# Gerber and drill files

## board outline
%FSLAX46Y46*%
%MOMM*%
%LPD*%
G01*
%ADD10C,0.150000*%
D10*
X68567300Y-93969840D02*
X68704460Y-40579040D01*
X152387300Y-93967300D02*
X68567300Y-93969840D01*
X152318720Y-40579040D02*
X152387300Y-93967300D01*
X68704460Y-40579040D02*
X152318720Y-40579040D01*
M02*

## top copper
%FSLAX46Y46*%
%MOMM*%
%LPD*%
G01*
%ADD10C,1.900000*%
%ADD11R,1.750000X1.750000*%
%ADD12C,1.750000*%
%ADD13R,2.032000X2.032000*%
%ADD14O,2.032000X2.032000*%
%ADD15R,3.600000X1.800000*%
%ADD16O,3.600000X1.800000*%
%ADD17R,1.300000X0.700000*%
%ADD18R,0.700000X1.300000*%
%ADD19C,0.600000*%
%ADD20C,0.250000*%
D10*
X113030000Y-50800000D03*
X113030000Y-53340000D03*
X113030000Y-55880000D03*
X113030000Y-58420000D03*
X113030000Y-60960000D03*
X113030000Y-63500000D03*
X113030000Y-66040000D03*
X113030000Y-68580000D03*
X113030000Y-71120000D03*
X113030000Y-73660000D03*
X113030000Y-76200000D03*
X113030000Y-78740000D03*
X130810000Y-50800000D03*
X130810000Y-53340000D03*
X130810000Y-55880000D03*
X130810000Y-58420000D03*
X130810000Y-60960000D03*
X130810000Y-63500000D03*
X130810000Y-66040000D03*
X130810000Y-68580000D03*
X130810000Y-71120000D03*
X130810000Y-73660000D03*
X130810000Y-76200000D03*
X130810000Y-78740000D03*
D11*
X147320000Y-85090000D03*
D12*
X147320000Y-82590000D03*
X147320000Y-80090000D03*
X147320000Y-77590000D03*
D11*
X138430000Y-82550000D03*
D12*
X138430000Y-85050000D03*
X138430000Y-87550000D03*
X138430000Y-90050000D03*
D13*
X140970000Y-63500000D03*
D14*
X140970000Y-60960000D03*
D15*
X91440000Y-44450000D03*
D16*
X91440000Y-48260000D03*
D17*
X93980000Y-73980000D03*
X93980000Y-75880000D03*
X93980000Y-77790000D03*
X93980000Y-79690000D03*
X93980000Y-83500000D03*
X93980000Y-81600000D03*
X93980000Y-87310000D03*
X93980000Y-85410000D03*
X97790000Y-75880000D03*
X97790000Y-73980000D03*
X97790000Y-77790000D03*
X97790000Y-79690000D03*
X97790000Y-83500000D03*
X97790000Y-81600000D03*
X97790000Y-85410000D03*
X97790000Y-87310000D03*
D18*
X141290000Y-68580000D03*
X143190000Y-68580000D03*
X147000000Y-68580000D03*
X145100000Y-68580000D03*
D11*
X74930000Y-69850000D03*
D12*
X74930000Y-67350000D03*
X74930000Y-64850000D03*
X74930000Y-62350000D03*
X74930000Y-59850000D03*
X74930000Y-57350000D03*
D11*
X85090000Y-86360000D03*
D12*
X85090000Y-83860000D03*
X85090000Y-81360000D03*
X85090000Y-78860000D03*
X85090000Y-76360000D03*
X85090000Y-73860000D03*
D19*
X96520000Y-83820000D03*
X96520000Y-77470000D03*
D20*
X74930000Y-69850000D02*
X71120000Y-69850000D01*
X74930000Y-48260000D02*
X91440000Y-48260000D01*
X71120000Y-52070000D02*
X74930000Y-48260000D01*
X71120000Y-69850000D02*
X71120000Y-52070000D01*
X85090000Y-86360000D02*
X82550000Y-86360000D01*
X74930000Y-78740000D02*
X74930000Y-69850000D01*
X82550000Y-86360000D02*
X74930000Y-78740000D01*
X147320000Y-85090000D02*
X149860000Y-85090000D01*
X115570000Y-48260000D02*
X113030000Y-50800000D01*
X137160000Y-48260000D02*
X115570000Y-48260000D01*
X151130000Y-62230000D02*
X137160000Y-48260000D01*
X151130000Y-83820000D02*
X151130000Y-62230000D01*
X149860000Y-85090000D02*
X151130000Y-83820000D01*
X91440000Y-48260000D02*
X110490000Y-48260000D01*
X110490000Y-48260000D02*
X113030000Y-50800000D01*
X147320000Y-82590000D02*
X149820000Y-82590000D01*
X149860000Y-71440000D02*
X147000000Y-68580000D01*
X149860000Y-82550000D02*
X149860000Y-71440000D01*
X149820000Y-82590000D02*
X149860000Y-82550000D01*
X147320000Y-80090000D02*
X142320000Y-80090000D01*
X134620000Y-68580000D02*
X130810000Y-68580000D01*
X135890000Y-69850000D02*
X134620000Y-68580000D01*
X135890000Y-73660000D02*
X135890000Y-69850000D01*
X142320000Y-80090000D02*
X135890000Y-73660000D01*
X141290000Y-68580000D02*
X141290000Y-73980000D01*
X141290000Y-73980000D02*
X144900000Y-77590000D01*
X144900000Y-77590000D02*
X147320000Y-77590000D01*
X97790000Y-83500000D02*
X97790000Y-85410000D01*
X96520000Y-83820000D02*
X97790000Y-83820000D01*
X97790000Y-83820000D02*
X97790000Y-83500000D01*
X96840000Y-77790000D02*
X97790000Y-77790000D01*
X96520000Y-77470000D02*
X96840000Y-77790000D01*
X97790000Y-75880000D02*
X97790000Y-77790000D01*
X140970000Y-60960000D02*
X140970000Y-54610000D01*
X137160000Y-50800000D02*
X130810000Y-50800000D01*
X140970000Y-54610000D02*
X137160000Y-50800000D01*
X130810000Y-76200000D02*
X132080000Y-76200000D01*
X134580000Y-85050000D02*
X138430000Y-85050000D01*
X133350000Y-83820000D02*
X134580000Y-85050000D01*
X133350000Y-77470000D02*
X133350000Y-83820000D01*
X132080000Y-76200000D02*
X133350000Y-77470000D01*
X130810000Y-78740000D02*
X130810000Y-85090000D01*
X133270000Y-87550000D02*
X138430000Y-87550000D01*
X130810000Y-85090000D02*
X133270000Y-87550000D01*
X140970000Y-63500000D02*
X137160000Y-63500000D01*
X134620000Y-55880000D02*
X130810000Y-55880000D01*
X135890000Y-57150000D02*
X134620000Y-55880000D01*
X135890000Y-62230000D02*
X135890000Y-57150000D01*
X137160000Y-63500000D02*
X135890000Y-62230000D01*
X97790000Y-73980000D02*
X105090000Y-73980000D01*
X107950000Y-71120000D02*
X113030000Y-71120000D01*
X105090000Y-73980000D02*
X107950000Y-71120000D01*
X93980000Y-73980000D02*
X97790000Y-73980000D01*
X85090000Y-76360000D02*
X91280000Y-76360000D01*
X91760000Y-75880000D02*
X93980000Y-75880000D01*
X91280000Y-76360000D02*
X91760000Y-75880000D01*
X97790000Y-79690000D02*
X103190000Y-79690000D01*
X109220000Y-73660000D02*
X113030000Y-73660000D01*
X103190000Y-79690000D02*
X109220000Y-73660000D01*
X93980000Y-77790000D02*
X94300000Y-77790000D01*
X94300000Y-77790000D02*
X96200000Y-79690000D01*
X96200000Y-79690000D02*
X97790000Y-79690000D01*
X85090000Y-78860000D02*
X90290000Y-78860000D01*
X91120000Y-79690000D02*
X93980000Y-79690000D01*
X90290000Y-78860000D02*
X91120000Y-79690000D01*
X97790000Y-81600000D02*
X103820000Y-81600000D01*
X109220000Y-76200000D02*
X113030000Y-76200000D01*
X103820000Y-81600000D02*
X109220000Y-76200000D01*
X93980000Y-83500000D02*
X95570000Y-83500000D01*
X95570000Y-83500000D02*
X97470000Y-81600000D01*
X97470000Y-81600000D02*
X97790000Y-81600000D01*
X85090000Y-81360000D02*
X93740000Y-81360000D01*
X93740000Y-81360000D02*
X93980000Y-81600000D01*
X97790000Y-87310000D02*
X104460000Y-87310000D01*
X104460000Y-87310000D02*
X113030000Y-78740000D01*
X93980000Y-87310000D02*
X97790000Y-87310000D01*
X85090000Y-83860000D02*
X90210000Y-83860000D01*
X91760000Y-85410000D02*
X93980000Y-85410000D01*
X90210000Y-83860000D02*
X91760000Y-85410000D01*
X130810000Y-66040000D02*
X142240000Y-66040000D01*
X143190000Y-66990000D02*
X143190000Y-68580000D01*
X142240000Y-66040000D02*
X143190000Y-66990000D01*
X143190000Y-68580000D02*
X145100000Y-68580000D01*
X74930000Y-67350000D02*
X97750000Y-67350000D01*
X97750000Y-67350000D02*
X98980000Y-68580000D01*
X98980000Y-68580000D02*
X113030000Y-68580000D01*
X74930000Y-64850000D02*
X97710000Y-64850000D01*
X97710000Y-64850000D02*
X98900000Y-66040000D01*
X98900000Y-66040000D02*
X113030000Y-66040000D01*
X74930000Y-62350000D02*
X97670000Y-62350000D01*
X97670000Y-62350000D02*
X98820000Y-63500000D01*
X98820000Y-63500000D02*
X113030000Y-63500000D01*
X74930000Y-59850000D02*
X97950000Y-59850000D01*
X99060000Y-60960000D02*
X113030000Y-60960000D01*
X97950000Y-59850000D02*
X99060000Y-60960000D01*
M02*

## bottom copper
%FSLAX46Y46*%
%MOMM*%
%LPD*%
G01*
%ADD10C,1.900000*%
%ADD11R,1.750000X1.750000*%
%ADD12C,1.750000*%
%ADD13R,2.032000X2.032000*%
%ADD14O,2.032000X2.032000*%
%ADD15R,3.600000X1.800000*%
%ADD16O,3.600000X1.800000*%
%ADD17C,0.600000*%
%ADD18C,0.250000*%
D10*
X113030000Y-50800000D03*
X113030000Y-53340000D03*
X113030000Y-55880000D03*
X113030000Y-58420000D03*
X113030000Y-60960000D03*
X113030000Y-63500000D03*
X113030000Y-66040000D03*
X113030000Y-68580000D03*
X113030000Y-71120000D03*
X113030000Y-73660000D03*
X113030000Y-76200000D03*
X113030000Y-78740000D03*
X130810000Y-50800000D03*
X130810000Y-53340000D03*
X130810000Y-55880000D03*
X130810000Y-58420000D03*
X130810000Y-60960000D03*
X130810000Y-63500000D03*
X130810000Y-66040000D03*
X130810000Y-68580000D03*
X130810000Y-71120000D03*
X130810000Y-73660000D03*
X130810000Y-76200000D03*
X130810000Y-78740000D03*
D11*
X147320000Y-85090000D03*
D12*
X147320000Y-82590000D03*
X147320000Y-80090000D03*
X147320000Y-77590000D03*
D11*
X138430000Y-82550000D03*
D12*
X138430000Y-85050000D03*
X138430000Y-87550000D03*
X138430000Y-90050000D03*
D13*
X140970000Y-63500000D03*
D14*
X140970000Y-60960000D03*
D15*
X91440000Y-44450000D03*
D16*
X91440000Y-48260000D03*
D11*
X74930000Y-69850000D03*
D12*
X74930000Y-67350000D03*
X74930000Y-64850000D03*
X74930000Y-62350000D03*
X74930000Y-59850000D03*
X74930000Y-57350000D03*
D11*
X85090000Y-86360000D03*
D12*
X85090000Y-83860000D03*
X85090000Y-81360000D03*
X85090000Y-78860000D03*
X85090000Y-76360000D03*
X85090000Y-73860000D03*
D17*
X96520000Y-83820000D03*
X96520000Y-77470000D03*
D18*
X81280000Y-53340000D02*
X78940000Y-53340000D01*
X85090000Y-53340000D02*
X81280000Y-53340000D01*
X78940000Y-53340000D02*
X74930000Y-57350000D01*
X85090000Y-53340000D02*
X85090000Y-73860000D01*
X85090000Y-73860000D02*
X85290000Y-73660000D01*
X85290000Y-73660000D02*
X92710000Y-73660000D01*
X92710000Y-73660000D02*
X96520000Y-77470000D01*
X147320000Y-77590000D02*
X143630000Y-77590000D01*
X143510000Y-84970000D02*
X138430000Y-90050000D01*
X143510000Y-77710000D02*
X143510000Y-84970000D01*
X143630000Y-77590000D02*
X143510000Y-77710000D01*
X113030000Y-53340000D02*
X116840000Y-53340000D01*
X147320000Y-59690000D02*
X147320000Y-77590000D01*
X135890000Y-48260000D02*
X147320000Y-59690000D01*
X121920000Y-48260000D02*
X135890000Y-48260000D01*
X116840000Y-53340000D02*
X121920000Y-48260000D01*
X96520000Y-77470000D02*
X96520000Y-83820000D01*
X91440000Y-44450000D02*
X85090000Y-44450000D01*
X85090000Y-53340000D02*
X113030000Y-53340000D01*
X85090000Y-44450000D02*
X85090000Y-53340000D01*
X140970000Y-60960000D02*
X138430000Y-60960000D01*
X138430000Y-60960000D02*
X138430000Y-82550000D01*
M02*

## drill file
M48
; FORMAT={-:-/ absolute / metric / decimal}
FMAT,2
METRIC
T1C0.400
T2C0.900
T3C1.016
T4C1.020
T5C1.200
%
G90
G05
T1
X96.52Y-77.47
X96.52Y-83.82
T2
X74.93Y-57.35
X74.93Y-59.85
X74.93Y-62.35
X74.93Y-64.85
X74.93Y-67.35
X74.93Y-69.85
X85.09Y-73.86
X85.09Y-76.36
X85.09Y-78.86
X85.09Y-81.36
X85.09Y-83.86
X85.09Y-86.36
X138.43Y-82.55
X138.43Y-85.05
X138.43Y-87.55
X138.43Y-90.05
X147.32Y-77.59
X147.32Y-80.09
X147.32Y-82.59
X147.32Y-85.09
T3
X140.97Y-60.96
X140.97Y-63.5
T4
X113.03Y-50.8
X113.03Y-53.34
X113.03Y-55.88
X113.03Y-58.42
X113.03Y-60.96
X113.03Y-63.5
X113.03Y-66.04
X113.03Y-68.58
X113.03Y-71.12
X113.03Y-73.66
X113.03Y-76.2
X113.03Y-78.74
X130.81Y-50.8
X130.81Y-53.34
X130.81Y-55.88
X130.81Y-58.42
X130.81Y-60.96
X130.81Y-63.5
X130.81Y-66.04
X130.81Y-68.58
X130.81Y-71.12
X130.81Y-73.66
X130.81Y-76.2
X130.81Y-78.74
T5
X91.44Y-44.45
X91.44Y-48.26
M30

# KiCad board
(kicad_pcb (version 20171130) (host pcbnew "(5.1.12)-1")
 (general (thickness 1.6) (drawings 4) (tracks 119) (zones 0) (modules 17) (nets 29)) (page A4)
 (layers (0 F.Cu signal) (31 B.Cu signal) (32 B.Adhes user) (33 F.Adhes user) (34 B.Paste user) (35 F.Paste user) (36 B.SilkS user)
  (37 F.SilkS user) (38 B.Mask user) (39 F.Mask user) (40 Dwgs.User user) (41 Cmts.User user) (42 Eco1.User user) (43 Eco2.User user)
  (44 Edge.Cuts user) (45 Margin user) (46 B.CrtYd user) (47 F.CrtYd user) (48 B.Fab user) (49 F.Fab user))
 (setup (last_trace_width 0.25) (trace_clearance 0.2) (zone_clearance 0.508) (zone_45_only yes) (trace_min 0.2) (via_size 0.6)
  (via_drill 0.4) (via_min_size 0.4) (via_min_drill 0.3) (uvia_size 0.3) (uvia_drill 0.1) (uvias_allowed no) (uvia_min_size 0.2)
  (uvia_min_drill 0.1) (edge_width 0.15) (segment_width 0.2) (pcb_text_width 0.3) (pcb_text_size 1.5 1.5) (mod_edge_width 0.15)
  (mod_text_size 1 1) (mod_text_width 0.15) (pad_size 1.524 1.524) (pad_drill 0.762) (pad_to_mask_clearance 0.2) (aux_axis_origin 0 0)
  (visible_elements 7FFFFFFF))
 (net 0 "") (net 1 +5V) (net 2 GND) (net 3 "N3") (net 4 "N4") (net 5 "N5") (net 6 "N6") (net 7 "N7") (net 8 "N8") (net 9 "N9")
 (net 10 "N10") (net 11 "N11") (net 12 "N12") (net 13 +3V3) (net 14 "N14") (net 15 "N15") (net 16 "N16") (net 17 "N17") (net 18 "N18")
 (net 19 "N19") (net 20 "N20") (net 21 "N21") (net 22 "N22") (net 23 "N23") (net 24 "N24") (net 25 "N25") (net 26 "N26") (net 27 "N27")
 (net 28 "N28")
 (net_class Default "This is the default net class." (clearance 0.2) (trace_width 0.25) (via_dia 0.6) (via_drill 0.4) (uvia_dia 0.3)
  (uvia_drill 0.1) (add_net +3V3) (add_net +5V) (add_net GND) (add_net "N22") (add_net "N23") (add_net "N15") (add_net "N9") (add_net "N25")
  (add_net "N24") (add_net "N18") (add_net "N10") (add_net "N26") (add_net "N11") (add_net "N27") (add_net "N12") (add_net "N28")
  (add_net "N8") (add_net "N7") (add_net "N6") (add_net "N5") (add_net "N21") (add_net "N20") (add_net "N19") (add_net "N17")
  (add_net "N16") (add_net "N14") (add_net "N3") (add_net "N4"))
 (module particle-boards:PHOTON (layer F.Cu) (at 121.92 66.04)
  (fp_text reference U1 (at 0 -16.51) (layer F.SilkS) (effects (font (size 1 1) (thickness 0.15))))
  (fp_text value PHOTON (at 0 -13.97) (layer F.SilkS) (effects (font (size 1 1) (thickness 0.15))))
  (pad 1 thru_hole circle (at -8.89 -15.24) (size 1.9 1.9) (drill 1.02) (layers *.Cu *.Mask F.SilkS) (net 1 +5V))
  (pad 2 thru_hole circle (at -8.89 -12.7) (size 1.9 1.9) (drill 1.02) (layers *.Cu *.Mask F.SilkS) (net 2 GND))
  (pad 3 thru_hole circle (at -8.89 -10.16) (size 1.9 1.9) (drill 1.02) (layers *.Cu *.Mask F.SilkS) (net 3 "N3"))
  (pad 4 thru_hole circle (at -8.89 -7.62) (size 1.9 1.9) (drill 1.02) (layers *.Cu *.Mask F.SilkS) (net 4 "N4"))
  (pad 5 thru_hole circle (at -8.89 -5.08) (size 1.9 1.9) (drill 1.02) (layers *.Cu *.Mask F.SilkS) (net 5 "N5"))
  (pad 6 thru_hole circle (at -8.89 -2.54) (size 1.9 1.9) (drill 1.02) (layers *.Cu *.Mask F.SilkS) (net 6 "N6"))
  (pad 7 thru_hole circle (at -8.89 0) (size 1.9 1.9) (drill 1.02) (layers *.Cu *.Mask F.SilkS) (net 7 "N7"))
  (pad 8 thru_hole circle (at -8.89 2.54) (size 1.9 1.9) (drill 1.02) (layers *.Cu *.Mask F.SilkS) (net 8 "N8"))
  (pad 9 thru_hole circle (at -8.89 5.08) (size 1.9 1.9) (drill 1.02) (layers *.Cu *.Mask F.SilkS) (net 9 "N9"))
  (pad 10 thru_hole circle (at -8.89 7.62) (size 1.9 1.9) (drill 1.02) (layers *.Cu *.Mask F.SilkS) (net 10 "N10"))
  (pad 11 thru_hole circle (at -8.89 10.16) (size 1.9 1.9) (drill 1.02) (layers *.Cu *.Mask F.SilkS) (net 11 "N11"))
  (pad 12 thru_hole circle (at -8.89 12.7) (size 1.9 1.9) (drill 1.02) (layers *.Cu *.Mask F.SilkS) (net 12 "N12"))
  (pad 24 thru_hole circle (at 8.89 -15.24) (size 1.9 1.9) (drill 1.02) (layers *.Cu *.Mask F.SilkS) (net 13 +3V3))
  (pad 23 thru_hole circle (at 8.89 -12.7) (size 1.9 1.9) (drill 1.02) (layers *.Cu *.Mask F.SilkS) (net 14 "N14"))
  (pad 22 thru_hole circle (at 8.89 -10.16) (size 1.9 1.9) (drill 1.02) (layers *.Cu *.Mask F.SilkS) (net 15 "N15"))
  (pad 21 thru_hole circle (at 8.89 -7.62) (size 1.9 1.9) (drill 1.02) (layers *.Cu *.Mask F.SilkS))
  (pad 20 thru_hole circle (at 8.89 -5.08) (size 1.9 1.9) (drill 1.02) (layers *.Cu *.Mask F.SilkS) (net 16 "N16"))
  (pad 19 thru_hole circle (at 8.89 -2.54) (size 1.9 1.9) (drill 1.02) (layers *.Cu *.Mask F.SilkS) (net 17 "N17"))
  (pad 18 thru_hole circle (at 8.89 0) (size 1.9 1.9) (drill 1.02) (layers *.Cu *.Mask F.SilkS) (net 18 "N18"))
  (pad 17 thru_hole circle (at 8.89 2.54) (size 1.9 1.9) (drill 1.02) (layers *.Cu *.Mask F.SilkS) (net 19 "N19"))
  (pad 16 thru_hole circle (at 8.89 5.08) (size 1.9 1.9) (drill 1.02) (layers *.Cu *.Mask F.SilkS) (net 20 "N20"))
  (pad 15 thru_hole circle (at 8.89 7.62) (size 1.9 1.9) (drill 1.02) (layers *.Cu *.Mask F.SilkS) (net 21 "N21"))
  (pad 14 thru_hole circle (at 8.89 10.16) (size 1.9 1.9) (drill 1.02) (layers *.Cu *.Mask F.SilkS) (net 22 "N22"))
  (pad 13 thru_hole circle (at 8.89 12.7) (size 1.9 1.9) (drill 1.02) (layers *.Cu *.Mask F.SilkS) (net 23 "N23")))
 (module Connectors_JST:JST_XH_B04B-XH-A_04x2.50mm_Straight (layer F.Cu) (at 147.32 85.09 90)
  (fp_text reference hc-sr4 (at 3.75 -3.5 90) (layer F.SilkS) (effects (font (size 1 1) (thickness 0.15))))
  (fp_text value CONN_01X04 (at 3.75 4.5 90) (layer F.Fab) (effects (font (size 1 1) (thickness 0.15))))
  (pad 1 thru_hole rect (at 0 0 90) (size 1.75 1.75) (drill 0.9) (layers *.Cu *.Mask) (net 1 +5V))
  (pad 2 thru_hole circle (at 2.5 0 90) (size 1.75 1.75) (drill 0.9) (layers *.Cu *.Mask) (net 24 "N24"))
  (pad 3 thru_hole circle (at 5 0 90) (size 1.75 1.75) (drill 0.9) (layers *.Cu *.Mask) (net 19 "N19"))
  (pad 4 thru_hole circle (at 7.5 0 90) (size 1.75 1.75) (drill 0.9) (layers *.Cu *.Mask) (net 2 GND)))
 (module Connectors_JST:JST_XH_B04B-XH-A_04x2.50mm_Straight (layer F.Cu) (at 138.43 82.55 270)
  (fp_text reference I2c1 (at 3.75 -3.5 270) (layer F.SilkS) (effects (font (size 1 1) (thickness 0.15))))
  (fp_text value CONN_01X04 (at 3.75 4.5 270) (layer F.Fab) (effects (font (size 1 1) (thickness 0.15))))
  (pad 1 thru_hole rect (at 0 0 270) (size 1.75 1.75) (drill 0.9) (layers *.Cu *.Mask) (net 13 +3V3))
  (pad 2 thru_hole circle (at 2.5 0 270) (size 1.75 1.75) (drill 0.9) (layers *.Cu *.Mask) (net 22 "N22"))
  (pad 3 thru_hole circle (at 5 0 270) (size 1.75 1.75) (drill 0.9) (layers *.Cu *.Mask) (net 23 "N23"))
  (pad 4 thru_hole circle (at 7.5 0 270) (size 1.75 1.75) (drill 0.9) (layers *.Cu *.Mask) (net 2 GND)))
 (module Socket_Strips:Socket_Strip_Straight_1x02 (layer F.Cu) (at 140.97 63.5 90)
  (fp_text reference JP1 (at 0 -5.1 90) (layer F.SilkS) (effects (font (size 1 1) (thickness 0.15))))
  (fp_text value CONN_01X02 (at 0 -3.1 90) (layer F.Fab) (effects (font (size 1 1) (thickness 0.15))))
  (pad 1 thru_hole rect (at 0 0 90) (size 2.032 2.032) (drill 1.016) (layers *.Cu *.Mask F.SilkS) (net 15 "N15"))
  (pad 2 thru_hole oval (at 2.54 0 90) (size 2.032 2.032) (drill 1.016) (layers *.Cu *.Mask F.SilkS) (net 13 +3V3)))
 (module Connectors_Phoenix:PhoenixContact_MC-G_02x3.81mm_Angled (layer F.Cu) (at 91.44 44.45 270)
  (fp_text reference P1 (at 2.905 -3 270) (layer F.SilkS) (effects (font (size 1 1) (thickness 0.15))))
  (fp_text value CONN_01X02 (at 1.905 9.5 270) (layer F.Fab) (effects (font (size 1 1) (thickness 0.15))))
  (pad 1 thru_hole rect (at 0 0 270) (size 1.8 3.6) (drill 1.2) (layers *.Cu *.Mask) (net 2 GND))
  (pad 2 thru_hole oval (at 3.81 0 270) (size 1.8 3.6) (drill 1.2) (layers *.Cu *.Mask) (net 1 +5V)))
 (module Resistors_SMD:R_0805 (layer F.Cu) (at 93.98 74.93 270)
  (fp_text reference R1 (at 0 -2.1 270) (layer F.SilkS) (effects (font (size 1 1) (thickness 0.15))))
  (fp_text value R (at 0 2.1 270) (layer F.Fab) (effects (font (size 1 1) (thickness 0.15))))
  (pad 1 smd rect (at -0.95 0 270) (size 0.7 1.3) (layers F.Cu F.Paste F.Mask) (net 9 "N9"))
  (pad 2 smd rect (at 0.95 0 270) (size 0.7 1.3) (layers F.Cu F.Paste F.Mask) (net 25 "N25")))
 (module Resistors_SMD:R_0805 (layer F.Cu) (at 93.98 78.74 270)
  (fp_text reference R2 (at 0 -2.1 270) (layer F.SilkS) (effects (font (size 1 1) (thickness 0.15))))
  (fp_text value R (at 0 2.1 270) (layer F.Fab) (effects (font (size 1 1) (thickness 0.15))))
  (pad 1 smd rect (at -0.95 0 270) (size 0.7 1.3) (layers F.Cu F.Paste F.Mask) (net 10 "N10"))
  (pad 2 smd rect (at 0.95 0 270) (size 0.7 1.3) (layers F.Cu F.Paste F.Mask) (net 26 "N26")))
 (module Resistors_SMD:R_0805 (layer F.Cu) (at 93.98 82.55 90)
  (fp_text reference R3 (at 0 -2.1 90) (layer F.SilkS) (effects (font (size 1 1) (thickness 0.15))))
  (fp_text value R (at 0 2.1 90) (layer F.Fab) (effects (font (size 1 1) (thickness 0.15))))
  (pad 1 smd rect (at -0.95 0 90) (size 0.7 1.3) (layers F.Cu F.Paste F.Mask) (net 11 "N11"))
  (pad 2 smd rect (at 0.95 0 90) (size 0.7 1.3) (layers F.Cu F.Paste F.Mask) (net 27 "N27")))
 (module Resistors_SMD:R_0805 (layer F.Cu) (at 93.98 86.36 90)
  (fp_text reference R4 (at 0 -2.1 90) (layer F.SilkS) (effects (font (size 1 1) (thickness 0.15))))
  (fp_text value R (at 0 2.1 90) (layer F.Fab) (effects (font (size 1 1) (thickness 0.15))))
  (pad 1 smd rect (at -0.95 0 90) (size 0.7 1.3) (layers F.Cu F.Paste F.Mask) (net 12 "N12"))
  (pad 2 smd rect (at 0.95 0 90) (size 0.7 1.3) (layers F.Cu F.Paste F.Mask) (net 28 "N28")))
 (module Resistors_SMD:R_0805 (layer F.Cu) (at 97.79 74.93 90)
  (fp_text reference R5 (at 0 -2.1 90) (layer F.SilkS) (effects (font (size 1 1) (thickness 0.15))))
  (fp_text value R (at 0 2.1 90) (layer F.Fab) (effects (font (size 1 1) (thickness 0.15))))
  (pad 1 smd rect (at -0.95 0 90) (size 0.7 1.3) (layers F.Cu F.Paste F.Mask) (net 2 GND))
  (pad 2 smd rect (at 0.95 0 90) (size 0.7 1.3) (layers F.Cu F.Paste F.Mask) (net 9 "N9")))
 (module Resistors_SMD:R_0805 (layer F.Cu) (at 97.79 78.74 270)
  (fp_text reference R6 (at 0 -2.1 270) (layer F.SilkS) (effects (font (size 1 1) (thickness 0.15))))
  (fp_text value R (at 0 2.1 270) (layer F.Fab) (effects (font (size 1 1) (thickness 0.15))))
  (pad 1 smd rect (at -0.95 0 270) (size 0.7 1.3) (layers F.Cu F.Paste F.Mask) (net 2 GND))
  (pad 2 smd rect (at 0.95 0 270) (size 0.7 1.3) (layers F.Cu F.Paste F.Mask) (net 10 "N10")))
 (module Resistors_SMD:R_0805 (layer F.Cu) (at 97.79 82.55 90)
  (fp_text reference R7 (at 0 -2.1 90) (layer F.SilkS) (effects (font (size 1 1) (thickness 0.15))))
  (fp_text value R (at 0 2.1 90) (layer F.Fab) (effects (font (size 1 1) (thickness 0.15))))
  (pad 1 smd rect (at -0.95 0 90) (size 0.7 1.3) (layers F.Cu F.Paste F.Mask) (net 2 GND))
  (pad 2 smd rect (at 0.95 0 90) (size 0.7 1.3) (layers F.Cu F.Paste F.Mask) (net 11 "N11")))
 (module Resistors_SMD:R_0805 (layer F.Cu) (at 97.79 86.36 270)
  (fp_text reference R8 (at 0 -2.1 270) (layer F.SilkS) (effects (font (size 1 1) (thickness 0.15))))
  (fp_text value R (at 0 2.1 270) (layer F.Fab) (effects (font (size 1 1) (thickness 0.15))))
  (pad 1 smd rect (at -0.95 0 270) (size 0.7 1.3) (layers F.Cu F.Paste F.Mask) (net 2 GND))
  (pad 2 smd rect (at 0.95 0 270) (size 0.7 1.3) (layers F.Cu F.Paste F.Mask) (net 12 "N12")))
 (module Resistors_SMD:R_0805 (layer F.Cu) (at 142.24 68.58)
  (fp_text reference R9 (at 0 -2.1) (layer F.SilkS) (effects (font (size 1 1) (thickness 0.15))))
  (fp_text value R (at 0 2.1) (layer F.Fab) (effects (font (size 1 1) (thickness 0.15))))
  (pad 1 smd rect (at -0.95 0) (size 0.7 1.3) (layers F.Cu F.Paste F.Mask) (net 2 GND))
  (pad 2 smd rect (at 0.95 0) (size 0.7 1.3) (layers F.Cu F.Paste F.Mask) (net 18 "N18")))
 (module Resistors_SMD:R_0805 (layer F.Cu) (at 146.05 68.58 180)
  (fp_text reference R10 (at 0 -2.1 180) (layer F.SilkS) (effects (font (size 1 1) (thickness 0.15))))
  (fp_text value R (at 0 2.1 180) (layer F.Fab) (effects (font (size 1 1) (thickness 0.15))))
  (pad 1 smd rect (at -0.95 0 180) (size 0.7 1.3) (layers F.Cu F.Paste F.Mask) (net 24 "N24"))
  (pad 2 smd rect (at 0.95 0 180) (size 0.7 1.3) (layers F.Cu F.Paste F.Mask) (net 18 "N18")))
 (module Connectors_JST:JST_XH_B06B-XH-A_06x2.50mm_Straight (layer F.Cu) (at 74.93 69.85 90)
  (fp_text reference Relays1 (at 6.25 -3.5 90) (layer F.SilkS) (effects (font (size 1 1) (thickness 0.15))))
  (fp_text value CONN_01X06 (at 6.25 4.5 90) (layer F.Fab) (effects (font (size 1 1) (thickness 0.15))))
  (pad 1 thru_hole rect (at 0 0 90) (size 1.75 1.75) (drill 0.9) (layers *.Cu *.Mask) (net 1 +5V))
  (pad 2 thru_hole circle (at 2.5 0 90) (size 1.75 1.75) (drill 0.9) (layers *.Cu *.Mask) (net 8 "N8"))
  (pad 3 thru_hole circle (at 5 0 90) (size 1.75 1.75) (drill 0.9) (layers *.Cu *.Mask) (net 7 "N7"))
  (pad 4 thru_hole circle (at 7.5 0 90) (size 1.75 1.75) (drill 0.9) (layers *.Cu *.Mask) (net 6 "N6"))
  (pad 5 thru_hole circle (at 10 0 90) (size 1.75 1.75) (drill 0.9) (layers *.Cu *.Mask) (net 5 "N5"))
  (pad 6 thru_hole circle (at 12.5 0 90) (size 1.75 1.75) (drill 0.9) (layers *.Cu *.Mask) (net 2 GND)))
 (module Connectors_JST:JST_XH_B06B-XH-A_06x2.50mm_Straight (layer F.Cu) (at 85.09 86.36 90)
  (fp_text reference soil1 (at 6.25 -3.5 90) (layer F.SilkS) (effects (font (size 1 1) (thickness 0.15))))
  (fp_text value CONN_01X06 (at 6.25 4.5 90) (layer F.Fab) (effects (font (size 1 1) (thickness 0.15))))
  (pad 1 thru_hole rect (at 0 0 90) (size 1.75 1.75) (drill 0.9) (layers *.Cu *.Mask) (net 1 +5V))
  (pad 2 thru_hole circle (at 2.5 0 90) (size 1.75 1.75) (drill 0.9) (layers *.Cu *.Mask) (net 28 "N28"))
  (pad 3 thru_hole circle (at 5 0 90) (size 1.75 1.75) (drill 0.9) (layers *.Cu *.Mask) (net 27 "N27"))
  (pad 4 thru_hole circle (at 7.5 0 90) (size 1.75 1.75) (drill 0.9) (layers *.Cu *.Mask) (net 26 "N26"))
  (pad 5 thru_hole circle (at 10 0 90) (size 1.75 1.75) (drill 0.9) (layers *.Cu *.Mask) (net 25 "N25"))
  (pad 6 thru_hole circle (at 12.5 0 90) (size 1.75 1.75) (drill 0.9) (layers *.Cu *.Mask) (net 2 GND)))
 (gr_line (start 68.5673 93.96984) (end 68.70446 40.57904) (layer Edge.Cuts) (width 0.15))
 (gr_line (start 152.3873 93.9673) (end 68.5673 93.96984) (layer Edge.Cuts) (width 0.15))
 (gr_line (start 152.31872 40.57904) (end 152.3873 93.9673) (layer Edge.Cuts) (width 0.15))
 (gr_line (start 68.70446 40.57904) (end 152.31872 40.57904) (layer Edge.Cuts) (width 0.15))
 (segment (start 74.93 69.85) (end 71.12 69.85) (width 0.25) (layer F.Cu) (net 1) (status 400000))
 (segment (start 74.93 48.26) (end 91.44 48.26) (width 0.25) (layer F.Cu) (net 1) (status 800000))
 (segment (start 71.12 52.07) (end 74.93 48.26) (width 0.25) (layer F.Cu) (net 1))
 (segment (start 71.12 69.85) (end 71.12 52.07) (width 0.25) (layer F.Cu) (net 1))
 (segment (start 85.09 86.36) (end 82.55 86.36) (width 0.25) (layer F.Cu) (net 1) (status 400000))
 (segment (start 74.93 78.74) (end 74.93 69.85) (width 0.25) (layer F.Cu) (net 1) (status 800000))
 (segment (start 82.55 86.36) (end 74.93 78.74) (width 0.25) (layer F.Cu) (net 1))
 (segment (start 147.32 85.09) (end 149.86 85.09) (width 0.25) (layer F.Cu) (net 1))
 (segment (start 115.57 48.26) (end 113.03 50.8) (width 0.25) (layer F.Cu) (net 1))
 (segment (start 137.16 48.26) (end 115.57 48.26) (width 0.25) (layer F.Cu) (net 1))
 (segment (start 151.13 62.23) (end 137.16 48.26) (width 0.25) (layer F.Cu) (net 1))
 (segment (start 151.13 83.82) (end 151.13 62.23) (width 0.25) (layer F.Cu) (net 1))
 (segment (start 149.86 85.09) (end 151.13 83.82) (width 0.25) (layer F.Cu) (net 1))
 (segment (start 91.44 48.26) (end 110.49 48.26) (width 0.25) (layer F.Cu) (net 1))
 (segment (start 110.49 48.26) (end 113.03 50.8) (width 0.25) (layer F.Cu) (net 1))
 (segment (start 147.32 82.59) (end 149.82 82.59) (width 0.25) (layer F.Cu) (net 24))
 (segment (start 149.86 71.44) (end 147 68.58) (width 0.25) (layer F.Cu) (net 24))
 (segment (start 149.86 82.55) (end 149.86 71.44) (width 0.25) (layer F.Cu) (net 24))
 (segment (start 149.82 82.59) (end 149.86 82.55) (width 0.25) (layer F.Cu) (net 24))
 (segment (start 147.32 80.09) (end 142.32 80.09) (width 0.25) (layer F.Cu) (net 19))
 (segment (start 134.62 68.58) (end 130.81 68.58) (width 0.25) (layer F.Cu) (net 19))
 (segment (start 135.89 69.85) (end 134.62 68.58) (width 0.25) (layer F.Cu) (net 19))
 (segment (start 135.89 73.66) (end 135.89 69.85) (width 0.25) (layer F.Cu) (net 19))
 (segment (start 142.32 80.09) (end 135.89 73.66) (width 0.25) (layer F.Cu) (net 19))
 (segment (start 81.28 53.34) (end 78.94 53.34) (width 0.25) (layer B.Cu) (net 2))
 (segment (start 85.09 53.34) (end 81.28 53.34) (width 0.25) (layer B.Cu) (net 2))
 (segment (start 78.94 53.34) (end 74.93 57.35) (width 0.25) (layer B.Cu) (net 2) (status 800000))
 (segment (start 85.09 53.34) (end 85.09 73.86) (width 0.25) (layer B.Cu) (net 2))
 (segment (start 85.09 73.86) (end 85.29 73.66) (width 0.25) (layer B.Cu) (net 2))
 (segment (start 85.29 73.66) (end 92.71 73.66) (width 0.25) (layer B.Cu) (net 2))
 (segment (start 92.71 73.66) (end 96.52 77.47) (width 0.25) (layer B.Cu) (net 2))
 (segment (start 147.32 77.59) (end 143.63 77.59) (width 0.25) (layer B.Cu) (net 2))
 (segment (start 143.51 84.97) (end 138.43 90.05) (width 0.25) (layer B.Cu) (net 2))
 (segment (start 143.51 77.71) (end 143.51 84.97) (width 0.25) (layer B.Cu) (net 2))
 (segment (start 143.63 77.59) (end 143.51 77.71) (width 0.25) (layer B.Cu) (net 2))
 (segment (start 113.03 53.34) (end 116.84 53.34) (width 0.25) (layer B.Cu) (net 2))
 (segment (start 147.32 59.69) (end 147.32 77.59) (width 0.25) (layer B.Cu) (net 2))
 (segment (start 135.89 48.26) (end 147.32 59.69) (width 0.25) (layer B.Cu) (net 2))
 (segment (start 121.92 48.26) (end 135.89 48.26) (width 0.25) (layer B.Cu) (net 2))
 (segment (start 116.84 53.34) (end 121.92 48.26) (width 0.25) (layer B.Cu) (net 2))
 (segment (start 141.29 68.58) (end 141.29 73.98) (width 0.25) (layer F.Cu) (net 2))
 (segment (start 141.29 73.98) (end 144.9 77.59) (width 0.25) (layer F.Cu) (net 2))
 (segment (start 144.9 77.59) (end 147.32 77.59) (width 0.25) (layer F.Cu) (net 2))
 (segment (start 97.79 83.5) (end 97.79 85.41) (width 0.25) (layer F.Cu) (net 2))
 (segment (start 96.52 77.47) (end 96.52 83.82) (width 0.25) (layer B.Cu) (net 2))
 (segment (start 96.52 83.82) (end 97.79 83.82) (width 0.25) (layer F.Cu) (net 2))
 (segment (start 97.79 83.82) (end 97.79 83.5) (width 0.25) (layer F.Cu) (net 2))
 (segment (start 96.84 77.79) (end 97.79 77.79) (width 0.25) (layer F.Cu) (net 2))
 (segment (start 96.52 77.47) (end 96.84 77.79) (width 0.25) (layer F.Cu) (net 2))
 (segment (start 97.79 75.88) (end 97.79 77.79) (width 0.25) (layer F.Cu) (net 2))
 (segment (start 91.44 44.45) (end 85.09 44.45) (width 0.25) (layer B.Cu) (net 2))
 (segment (start 85.09 53.34) (end 113.03 53.34) (width 0.25) (layer B.Cu) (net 2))
 (segment (start 85.09 44.45) (end 85.09 53.34) (width 0.25) (layer B.Cu) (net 2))
 (segment (start 140.97 60.96) (end 138.43 60.96) (width 0.25) (layer B.Cu) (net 13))
 (segment (start 138.43 60.96) (end 138.43 82.55) (width 0.25) (layer B.Cu) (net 13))
 (segment (start 140.97 60.96) (end 140.97 54.61) (width 0.25) (layer F.Cu) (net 13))
 (segment (start 137.16 50.8) (end 130.81 50.8) (width 0.25) (layer F.Cu) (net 13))
 (segment (start 140.97 54.61) (end 137.16 50.8) (width 0.25) (layer F.Cu) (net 13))
 (segment (start 130.81 76.2) (end 132.08 76.2) (width 0.25) (layer F.Cu) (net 22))
 (segment (start 134.58 85.05) (end 138.43 85.05) (width 0.25) (layer F.Cu) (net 22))
 (segment (start 133.35 83.82) (end 134.58 85.05) (width 0.25) (layer F.Cu) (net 22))
 (segment (start 133.35 77.47) (end 133.35 83.82) (width 0.25) (layer F.Cu) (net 22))
 (segment (start 132.08 76.2) (end 133.35 77.47) (width 0.25) (layer F.Cu) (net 22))
 (segment (start 130.81 78.74) (end 130.81 85.09) (width 0.25) (layer F.Cu) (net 23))
 (segment (start 133.27 87.55) (end 138.43 87.55) (width 0.25) (layer F.Cu) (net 23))
 (segment (start 130.81 85.09) (end 133.27 87.55) (width 0.25) (layer F.Cu) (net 23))
 (segment (start 140.97 63.5) (end 137.16 63.5) (width 0.25) (layer F.Cu) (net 15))
 (segment (start 134.62 55.88) (end 130.81 55.88) (width 0.25) (layer F.Cu) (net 15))
 (segment (start 135.89 57.15) (end 134.62 55.88) (width 0.25) (layer F.Cu) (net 15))
 (segment (start 135.89 62.23) (end 135.89 57.15) (width 0.25) (layer F.Cu) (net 15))
 (segment (start 137.16 63.5) (end 135.89 62.23) (width 0.25) (layer F.Cu) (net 15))
 (segment (start 97.79 73.98) (end 105.09 73.98) (width 0.25) (layer F.Cu) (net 9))
 (segment (start 107.95 71.12) (end 113.03 71.12) (width 0.25) (layer F.Cu) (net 9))
 (segment (start 105.09 73.98) (end 107.95 71.12) (width 0.25) (layer F.Cu) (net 9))
 (segment (start 93.98 73.98) (end 97.79 73.98) (width 0.25) (layer F.Cu) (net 9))
 (segment (start 85.09 76.36) (end 91.28 76.36) (width 0.25) (layer F.Cu) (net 25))
 (segment (start 91.76 75.88) (end 93.98 75.88) (width 0.25) (layer F.Cu) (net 25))
 (segment (start 91.28 76.36) (end 91.76 75.88) (width 0.25) (layer F.Cu) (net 25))
 (segment (start 97.79 79.69) (end 103.19 79.69) (width 0.25) (layer F.Cu) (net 10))
 (segment (start 109.22 73.66) (end 113.03 73.66) (width 0.25) (layer F.Cu) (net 10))
 (segment (start 103.19 79.69) (end 109.22 73.66) (width 0.25) (layer F.Cu) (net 10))
 (segment (start 93.98 77.79) (end 94.3 77.79) (width 0.25) (layer F.Cu) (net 10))
 (segment (start 94.3 77.79) (end 96.2 79.69) (width 0.25) (layer F.Cu) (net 10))
 (segment (start 96.2 79.69) (end 97.79 79.69) (width 0.25) (layer F.Cu) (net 10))
 (segment (start 85.09 78.86) (end 90.29 78.86) (width 0.25) (layer F.Cu) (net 26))
 (segment (start 91.12 79.69) (end 93.98 79.69) (width 0.25) (layer F.Cu) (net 26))
 (segment (start 90.29 78.86) (end 91.12 79.69) (width 0.25) (layer F.Cu) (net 26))
 (segment (start 97.79 81.6) (end 103.82 81.6) (width 0.25) (layer F.Cu) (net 11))
 (segment (start 109.22 76.2) (end 113.03 76.2) (width 0.25) (layer F.Cu) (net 11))
 (segment (start 103.82 81.6) (end 109.22 76.2) (width 0.25) (layer F.Cu) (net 11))
 (segment (start 93.98 83.5) (end 95.57 83.5) (width 0.25) (layer F.Cu) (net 11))
 (segment (start 95.57 83.5) (end 97.47 81.6) (width 0.25) (layer F.Cu) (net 11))
 (segment (start 97.47 81.6) (end 97.79 81.6) (width 0.25) (layer F.Cu) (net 11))
 (segment (start 85.09 81.36) (end 93.74 81.36) (width 0.25) (layer F.Cu) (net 27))
 (segment (start 93.74 81.36) (end 93.98 81.6) (width 0.25) (layer F.Cu) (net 27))
 (segment (start 97.79 87.31) (end 104.46 87.31) (width 0.25) (layer F.Cu) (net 12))
 (segment (start 104.46 87.31) (end 113.03 78.74) (width 0.25) (layer F.Cu) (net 12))
 (segment (start 93.98 87.31) (end 97.79 87.31) (width 0.25) (layer F.Cu) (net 12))
 (segment (start 85.09 83.86) (end 90.21 83.86) (width 0.25) (layer F.Cu) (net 28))
 (segment (start 91.76 85.41) (end 93.98 85.41) (width 0.25) (layer F.Cu) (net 28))
 (segment (start 90.21 83.86) (end 91.76 85.41) (width 0.25) (layer F.Cu) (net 28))
 (segment (start 130.81 66.04) (end 142.24 66.04) (width 0.25) (layer F.Cu) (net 18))
 (segment (start 143.19 66.99) (end 143.19 68.58) (width 0.25) (layer F.Cu) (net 18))
 (segment (start 142.24 66.04) (end 143.19 66.99) (width 0.25) (layer F.Cu) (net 18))
 (segment (start 143.19 68.58) (end 145.1 68.58) (width 0.25) (layer F.Cu) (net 18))
 (segment (start 74.93 67.35) (end 97.75 67.35) (width 0.25) (layer F.Cu) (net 8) (status 400000))
 (segment (start 97.75 67.35) (end 98.98 68.58) (width 0.25) (layer F.Cu) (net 8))
 (segment (start 98.98 68.58) (end 113.03 68.58) (width 0.25) (layer F.Cu) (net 8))
 (segment (start 74.93 64.85) (end 97.71 64.85) (width 0.25) (layer F.Cu) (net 7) (status 400000))
 (segment (start 97.71 64.85) (end 98.9 66.04) (width 0.25) (layer F.Cu) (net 7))
 (segment (start 98.9 66.04) (end 113.03 66.04) (width 0.25) (layer F.Cu) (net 7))
 (segment (start 74.93 62.35) (end 97.67 62.35) (width 0.25) (layer F.Cu) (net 6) (status 400000))
 (segment (start 97.67 62.35) (end 98.82 63.5) (width 0.25) (layer F.Cu) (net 6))
 (segment (start 98.82 63.5) (end 113.03 63.5) (width 0.25) (layer F.Cu) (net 6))
 (segment (start 74.93 59.85) (end 97.95 59.85) (width 0.25) (layer F.Cu) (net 5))
 (segment (start 99.06 60.96) (end 113.03 60.96) (width 0.25) (layer F.Cu) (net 5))
 (segment (start 97.95 59.85) (end 99.06 60.96) (width 0.25) (layer F.Cu) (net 5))
 (via (at 96.52 83.82) (size 0.6) (drill 0.4) (layers F.Cu B.Cu) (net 2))
 (via (at 96.52 77.47) (size 0.6) (drill 0.4) (layers F.Cu B.Cu) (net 2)))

